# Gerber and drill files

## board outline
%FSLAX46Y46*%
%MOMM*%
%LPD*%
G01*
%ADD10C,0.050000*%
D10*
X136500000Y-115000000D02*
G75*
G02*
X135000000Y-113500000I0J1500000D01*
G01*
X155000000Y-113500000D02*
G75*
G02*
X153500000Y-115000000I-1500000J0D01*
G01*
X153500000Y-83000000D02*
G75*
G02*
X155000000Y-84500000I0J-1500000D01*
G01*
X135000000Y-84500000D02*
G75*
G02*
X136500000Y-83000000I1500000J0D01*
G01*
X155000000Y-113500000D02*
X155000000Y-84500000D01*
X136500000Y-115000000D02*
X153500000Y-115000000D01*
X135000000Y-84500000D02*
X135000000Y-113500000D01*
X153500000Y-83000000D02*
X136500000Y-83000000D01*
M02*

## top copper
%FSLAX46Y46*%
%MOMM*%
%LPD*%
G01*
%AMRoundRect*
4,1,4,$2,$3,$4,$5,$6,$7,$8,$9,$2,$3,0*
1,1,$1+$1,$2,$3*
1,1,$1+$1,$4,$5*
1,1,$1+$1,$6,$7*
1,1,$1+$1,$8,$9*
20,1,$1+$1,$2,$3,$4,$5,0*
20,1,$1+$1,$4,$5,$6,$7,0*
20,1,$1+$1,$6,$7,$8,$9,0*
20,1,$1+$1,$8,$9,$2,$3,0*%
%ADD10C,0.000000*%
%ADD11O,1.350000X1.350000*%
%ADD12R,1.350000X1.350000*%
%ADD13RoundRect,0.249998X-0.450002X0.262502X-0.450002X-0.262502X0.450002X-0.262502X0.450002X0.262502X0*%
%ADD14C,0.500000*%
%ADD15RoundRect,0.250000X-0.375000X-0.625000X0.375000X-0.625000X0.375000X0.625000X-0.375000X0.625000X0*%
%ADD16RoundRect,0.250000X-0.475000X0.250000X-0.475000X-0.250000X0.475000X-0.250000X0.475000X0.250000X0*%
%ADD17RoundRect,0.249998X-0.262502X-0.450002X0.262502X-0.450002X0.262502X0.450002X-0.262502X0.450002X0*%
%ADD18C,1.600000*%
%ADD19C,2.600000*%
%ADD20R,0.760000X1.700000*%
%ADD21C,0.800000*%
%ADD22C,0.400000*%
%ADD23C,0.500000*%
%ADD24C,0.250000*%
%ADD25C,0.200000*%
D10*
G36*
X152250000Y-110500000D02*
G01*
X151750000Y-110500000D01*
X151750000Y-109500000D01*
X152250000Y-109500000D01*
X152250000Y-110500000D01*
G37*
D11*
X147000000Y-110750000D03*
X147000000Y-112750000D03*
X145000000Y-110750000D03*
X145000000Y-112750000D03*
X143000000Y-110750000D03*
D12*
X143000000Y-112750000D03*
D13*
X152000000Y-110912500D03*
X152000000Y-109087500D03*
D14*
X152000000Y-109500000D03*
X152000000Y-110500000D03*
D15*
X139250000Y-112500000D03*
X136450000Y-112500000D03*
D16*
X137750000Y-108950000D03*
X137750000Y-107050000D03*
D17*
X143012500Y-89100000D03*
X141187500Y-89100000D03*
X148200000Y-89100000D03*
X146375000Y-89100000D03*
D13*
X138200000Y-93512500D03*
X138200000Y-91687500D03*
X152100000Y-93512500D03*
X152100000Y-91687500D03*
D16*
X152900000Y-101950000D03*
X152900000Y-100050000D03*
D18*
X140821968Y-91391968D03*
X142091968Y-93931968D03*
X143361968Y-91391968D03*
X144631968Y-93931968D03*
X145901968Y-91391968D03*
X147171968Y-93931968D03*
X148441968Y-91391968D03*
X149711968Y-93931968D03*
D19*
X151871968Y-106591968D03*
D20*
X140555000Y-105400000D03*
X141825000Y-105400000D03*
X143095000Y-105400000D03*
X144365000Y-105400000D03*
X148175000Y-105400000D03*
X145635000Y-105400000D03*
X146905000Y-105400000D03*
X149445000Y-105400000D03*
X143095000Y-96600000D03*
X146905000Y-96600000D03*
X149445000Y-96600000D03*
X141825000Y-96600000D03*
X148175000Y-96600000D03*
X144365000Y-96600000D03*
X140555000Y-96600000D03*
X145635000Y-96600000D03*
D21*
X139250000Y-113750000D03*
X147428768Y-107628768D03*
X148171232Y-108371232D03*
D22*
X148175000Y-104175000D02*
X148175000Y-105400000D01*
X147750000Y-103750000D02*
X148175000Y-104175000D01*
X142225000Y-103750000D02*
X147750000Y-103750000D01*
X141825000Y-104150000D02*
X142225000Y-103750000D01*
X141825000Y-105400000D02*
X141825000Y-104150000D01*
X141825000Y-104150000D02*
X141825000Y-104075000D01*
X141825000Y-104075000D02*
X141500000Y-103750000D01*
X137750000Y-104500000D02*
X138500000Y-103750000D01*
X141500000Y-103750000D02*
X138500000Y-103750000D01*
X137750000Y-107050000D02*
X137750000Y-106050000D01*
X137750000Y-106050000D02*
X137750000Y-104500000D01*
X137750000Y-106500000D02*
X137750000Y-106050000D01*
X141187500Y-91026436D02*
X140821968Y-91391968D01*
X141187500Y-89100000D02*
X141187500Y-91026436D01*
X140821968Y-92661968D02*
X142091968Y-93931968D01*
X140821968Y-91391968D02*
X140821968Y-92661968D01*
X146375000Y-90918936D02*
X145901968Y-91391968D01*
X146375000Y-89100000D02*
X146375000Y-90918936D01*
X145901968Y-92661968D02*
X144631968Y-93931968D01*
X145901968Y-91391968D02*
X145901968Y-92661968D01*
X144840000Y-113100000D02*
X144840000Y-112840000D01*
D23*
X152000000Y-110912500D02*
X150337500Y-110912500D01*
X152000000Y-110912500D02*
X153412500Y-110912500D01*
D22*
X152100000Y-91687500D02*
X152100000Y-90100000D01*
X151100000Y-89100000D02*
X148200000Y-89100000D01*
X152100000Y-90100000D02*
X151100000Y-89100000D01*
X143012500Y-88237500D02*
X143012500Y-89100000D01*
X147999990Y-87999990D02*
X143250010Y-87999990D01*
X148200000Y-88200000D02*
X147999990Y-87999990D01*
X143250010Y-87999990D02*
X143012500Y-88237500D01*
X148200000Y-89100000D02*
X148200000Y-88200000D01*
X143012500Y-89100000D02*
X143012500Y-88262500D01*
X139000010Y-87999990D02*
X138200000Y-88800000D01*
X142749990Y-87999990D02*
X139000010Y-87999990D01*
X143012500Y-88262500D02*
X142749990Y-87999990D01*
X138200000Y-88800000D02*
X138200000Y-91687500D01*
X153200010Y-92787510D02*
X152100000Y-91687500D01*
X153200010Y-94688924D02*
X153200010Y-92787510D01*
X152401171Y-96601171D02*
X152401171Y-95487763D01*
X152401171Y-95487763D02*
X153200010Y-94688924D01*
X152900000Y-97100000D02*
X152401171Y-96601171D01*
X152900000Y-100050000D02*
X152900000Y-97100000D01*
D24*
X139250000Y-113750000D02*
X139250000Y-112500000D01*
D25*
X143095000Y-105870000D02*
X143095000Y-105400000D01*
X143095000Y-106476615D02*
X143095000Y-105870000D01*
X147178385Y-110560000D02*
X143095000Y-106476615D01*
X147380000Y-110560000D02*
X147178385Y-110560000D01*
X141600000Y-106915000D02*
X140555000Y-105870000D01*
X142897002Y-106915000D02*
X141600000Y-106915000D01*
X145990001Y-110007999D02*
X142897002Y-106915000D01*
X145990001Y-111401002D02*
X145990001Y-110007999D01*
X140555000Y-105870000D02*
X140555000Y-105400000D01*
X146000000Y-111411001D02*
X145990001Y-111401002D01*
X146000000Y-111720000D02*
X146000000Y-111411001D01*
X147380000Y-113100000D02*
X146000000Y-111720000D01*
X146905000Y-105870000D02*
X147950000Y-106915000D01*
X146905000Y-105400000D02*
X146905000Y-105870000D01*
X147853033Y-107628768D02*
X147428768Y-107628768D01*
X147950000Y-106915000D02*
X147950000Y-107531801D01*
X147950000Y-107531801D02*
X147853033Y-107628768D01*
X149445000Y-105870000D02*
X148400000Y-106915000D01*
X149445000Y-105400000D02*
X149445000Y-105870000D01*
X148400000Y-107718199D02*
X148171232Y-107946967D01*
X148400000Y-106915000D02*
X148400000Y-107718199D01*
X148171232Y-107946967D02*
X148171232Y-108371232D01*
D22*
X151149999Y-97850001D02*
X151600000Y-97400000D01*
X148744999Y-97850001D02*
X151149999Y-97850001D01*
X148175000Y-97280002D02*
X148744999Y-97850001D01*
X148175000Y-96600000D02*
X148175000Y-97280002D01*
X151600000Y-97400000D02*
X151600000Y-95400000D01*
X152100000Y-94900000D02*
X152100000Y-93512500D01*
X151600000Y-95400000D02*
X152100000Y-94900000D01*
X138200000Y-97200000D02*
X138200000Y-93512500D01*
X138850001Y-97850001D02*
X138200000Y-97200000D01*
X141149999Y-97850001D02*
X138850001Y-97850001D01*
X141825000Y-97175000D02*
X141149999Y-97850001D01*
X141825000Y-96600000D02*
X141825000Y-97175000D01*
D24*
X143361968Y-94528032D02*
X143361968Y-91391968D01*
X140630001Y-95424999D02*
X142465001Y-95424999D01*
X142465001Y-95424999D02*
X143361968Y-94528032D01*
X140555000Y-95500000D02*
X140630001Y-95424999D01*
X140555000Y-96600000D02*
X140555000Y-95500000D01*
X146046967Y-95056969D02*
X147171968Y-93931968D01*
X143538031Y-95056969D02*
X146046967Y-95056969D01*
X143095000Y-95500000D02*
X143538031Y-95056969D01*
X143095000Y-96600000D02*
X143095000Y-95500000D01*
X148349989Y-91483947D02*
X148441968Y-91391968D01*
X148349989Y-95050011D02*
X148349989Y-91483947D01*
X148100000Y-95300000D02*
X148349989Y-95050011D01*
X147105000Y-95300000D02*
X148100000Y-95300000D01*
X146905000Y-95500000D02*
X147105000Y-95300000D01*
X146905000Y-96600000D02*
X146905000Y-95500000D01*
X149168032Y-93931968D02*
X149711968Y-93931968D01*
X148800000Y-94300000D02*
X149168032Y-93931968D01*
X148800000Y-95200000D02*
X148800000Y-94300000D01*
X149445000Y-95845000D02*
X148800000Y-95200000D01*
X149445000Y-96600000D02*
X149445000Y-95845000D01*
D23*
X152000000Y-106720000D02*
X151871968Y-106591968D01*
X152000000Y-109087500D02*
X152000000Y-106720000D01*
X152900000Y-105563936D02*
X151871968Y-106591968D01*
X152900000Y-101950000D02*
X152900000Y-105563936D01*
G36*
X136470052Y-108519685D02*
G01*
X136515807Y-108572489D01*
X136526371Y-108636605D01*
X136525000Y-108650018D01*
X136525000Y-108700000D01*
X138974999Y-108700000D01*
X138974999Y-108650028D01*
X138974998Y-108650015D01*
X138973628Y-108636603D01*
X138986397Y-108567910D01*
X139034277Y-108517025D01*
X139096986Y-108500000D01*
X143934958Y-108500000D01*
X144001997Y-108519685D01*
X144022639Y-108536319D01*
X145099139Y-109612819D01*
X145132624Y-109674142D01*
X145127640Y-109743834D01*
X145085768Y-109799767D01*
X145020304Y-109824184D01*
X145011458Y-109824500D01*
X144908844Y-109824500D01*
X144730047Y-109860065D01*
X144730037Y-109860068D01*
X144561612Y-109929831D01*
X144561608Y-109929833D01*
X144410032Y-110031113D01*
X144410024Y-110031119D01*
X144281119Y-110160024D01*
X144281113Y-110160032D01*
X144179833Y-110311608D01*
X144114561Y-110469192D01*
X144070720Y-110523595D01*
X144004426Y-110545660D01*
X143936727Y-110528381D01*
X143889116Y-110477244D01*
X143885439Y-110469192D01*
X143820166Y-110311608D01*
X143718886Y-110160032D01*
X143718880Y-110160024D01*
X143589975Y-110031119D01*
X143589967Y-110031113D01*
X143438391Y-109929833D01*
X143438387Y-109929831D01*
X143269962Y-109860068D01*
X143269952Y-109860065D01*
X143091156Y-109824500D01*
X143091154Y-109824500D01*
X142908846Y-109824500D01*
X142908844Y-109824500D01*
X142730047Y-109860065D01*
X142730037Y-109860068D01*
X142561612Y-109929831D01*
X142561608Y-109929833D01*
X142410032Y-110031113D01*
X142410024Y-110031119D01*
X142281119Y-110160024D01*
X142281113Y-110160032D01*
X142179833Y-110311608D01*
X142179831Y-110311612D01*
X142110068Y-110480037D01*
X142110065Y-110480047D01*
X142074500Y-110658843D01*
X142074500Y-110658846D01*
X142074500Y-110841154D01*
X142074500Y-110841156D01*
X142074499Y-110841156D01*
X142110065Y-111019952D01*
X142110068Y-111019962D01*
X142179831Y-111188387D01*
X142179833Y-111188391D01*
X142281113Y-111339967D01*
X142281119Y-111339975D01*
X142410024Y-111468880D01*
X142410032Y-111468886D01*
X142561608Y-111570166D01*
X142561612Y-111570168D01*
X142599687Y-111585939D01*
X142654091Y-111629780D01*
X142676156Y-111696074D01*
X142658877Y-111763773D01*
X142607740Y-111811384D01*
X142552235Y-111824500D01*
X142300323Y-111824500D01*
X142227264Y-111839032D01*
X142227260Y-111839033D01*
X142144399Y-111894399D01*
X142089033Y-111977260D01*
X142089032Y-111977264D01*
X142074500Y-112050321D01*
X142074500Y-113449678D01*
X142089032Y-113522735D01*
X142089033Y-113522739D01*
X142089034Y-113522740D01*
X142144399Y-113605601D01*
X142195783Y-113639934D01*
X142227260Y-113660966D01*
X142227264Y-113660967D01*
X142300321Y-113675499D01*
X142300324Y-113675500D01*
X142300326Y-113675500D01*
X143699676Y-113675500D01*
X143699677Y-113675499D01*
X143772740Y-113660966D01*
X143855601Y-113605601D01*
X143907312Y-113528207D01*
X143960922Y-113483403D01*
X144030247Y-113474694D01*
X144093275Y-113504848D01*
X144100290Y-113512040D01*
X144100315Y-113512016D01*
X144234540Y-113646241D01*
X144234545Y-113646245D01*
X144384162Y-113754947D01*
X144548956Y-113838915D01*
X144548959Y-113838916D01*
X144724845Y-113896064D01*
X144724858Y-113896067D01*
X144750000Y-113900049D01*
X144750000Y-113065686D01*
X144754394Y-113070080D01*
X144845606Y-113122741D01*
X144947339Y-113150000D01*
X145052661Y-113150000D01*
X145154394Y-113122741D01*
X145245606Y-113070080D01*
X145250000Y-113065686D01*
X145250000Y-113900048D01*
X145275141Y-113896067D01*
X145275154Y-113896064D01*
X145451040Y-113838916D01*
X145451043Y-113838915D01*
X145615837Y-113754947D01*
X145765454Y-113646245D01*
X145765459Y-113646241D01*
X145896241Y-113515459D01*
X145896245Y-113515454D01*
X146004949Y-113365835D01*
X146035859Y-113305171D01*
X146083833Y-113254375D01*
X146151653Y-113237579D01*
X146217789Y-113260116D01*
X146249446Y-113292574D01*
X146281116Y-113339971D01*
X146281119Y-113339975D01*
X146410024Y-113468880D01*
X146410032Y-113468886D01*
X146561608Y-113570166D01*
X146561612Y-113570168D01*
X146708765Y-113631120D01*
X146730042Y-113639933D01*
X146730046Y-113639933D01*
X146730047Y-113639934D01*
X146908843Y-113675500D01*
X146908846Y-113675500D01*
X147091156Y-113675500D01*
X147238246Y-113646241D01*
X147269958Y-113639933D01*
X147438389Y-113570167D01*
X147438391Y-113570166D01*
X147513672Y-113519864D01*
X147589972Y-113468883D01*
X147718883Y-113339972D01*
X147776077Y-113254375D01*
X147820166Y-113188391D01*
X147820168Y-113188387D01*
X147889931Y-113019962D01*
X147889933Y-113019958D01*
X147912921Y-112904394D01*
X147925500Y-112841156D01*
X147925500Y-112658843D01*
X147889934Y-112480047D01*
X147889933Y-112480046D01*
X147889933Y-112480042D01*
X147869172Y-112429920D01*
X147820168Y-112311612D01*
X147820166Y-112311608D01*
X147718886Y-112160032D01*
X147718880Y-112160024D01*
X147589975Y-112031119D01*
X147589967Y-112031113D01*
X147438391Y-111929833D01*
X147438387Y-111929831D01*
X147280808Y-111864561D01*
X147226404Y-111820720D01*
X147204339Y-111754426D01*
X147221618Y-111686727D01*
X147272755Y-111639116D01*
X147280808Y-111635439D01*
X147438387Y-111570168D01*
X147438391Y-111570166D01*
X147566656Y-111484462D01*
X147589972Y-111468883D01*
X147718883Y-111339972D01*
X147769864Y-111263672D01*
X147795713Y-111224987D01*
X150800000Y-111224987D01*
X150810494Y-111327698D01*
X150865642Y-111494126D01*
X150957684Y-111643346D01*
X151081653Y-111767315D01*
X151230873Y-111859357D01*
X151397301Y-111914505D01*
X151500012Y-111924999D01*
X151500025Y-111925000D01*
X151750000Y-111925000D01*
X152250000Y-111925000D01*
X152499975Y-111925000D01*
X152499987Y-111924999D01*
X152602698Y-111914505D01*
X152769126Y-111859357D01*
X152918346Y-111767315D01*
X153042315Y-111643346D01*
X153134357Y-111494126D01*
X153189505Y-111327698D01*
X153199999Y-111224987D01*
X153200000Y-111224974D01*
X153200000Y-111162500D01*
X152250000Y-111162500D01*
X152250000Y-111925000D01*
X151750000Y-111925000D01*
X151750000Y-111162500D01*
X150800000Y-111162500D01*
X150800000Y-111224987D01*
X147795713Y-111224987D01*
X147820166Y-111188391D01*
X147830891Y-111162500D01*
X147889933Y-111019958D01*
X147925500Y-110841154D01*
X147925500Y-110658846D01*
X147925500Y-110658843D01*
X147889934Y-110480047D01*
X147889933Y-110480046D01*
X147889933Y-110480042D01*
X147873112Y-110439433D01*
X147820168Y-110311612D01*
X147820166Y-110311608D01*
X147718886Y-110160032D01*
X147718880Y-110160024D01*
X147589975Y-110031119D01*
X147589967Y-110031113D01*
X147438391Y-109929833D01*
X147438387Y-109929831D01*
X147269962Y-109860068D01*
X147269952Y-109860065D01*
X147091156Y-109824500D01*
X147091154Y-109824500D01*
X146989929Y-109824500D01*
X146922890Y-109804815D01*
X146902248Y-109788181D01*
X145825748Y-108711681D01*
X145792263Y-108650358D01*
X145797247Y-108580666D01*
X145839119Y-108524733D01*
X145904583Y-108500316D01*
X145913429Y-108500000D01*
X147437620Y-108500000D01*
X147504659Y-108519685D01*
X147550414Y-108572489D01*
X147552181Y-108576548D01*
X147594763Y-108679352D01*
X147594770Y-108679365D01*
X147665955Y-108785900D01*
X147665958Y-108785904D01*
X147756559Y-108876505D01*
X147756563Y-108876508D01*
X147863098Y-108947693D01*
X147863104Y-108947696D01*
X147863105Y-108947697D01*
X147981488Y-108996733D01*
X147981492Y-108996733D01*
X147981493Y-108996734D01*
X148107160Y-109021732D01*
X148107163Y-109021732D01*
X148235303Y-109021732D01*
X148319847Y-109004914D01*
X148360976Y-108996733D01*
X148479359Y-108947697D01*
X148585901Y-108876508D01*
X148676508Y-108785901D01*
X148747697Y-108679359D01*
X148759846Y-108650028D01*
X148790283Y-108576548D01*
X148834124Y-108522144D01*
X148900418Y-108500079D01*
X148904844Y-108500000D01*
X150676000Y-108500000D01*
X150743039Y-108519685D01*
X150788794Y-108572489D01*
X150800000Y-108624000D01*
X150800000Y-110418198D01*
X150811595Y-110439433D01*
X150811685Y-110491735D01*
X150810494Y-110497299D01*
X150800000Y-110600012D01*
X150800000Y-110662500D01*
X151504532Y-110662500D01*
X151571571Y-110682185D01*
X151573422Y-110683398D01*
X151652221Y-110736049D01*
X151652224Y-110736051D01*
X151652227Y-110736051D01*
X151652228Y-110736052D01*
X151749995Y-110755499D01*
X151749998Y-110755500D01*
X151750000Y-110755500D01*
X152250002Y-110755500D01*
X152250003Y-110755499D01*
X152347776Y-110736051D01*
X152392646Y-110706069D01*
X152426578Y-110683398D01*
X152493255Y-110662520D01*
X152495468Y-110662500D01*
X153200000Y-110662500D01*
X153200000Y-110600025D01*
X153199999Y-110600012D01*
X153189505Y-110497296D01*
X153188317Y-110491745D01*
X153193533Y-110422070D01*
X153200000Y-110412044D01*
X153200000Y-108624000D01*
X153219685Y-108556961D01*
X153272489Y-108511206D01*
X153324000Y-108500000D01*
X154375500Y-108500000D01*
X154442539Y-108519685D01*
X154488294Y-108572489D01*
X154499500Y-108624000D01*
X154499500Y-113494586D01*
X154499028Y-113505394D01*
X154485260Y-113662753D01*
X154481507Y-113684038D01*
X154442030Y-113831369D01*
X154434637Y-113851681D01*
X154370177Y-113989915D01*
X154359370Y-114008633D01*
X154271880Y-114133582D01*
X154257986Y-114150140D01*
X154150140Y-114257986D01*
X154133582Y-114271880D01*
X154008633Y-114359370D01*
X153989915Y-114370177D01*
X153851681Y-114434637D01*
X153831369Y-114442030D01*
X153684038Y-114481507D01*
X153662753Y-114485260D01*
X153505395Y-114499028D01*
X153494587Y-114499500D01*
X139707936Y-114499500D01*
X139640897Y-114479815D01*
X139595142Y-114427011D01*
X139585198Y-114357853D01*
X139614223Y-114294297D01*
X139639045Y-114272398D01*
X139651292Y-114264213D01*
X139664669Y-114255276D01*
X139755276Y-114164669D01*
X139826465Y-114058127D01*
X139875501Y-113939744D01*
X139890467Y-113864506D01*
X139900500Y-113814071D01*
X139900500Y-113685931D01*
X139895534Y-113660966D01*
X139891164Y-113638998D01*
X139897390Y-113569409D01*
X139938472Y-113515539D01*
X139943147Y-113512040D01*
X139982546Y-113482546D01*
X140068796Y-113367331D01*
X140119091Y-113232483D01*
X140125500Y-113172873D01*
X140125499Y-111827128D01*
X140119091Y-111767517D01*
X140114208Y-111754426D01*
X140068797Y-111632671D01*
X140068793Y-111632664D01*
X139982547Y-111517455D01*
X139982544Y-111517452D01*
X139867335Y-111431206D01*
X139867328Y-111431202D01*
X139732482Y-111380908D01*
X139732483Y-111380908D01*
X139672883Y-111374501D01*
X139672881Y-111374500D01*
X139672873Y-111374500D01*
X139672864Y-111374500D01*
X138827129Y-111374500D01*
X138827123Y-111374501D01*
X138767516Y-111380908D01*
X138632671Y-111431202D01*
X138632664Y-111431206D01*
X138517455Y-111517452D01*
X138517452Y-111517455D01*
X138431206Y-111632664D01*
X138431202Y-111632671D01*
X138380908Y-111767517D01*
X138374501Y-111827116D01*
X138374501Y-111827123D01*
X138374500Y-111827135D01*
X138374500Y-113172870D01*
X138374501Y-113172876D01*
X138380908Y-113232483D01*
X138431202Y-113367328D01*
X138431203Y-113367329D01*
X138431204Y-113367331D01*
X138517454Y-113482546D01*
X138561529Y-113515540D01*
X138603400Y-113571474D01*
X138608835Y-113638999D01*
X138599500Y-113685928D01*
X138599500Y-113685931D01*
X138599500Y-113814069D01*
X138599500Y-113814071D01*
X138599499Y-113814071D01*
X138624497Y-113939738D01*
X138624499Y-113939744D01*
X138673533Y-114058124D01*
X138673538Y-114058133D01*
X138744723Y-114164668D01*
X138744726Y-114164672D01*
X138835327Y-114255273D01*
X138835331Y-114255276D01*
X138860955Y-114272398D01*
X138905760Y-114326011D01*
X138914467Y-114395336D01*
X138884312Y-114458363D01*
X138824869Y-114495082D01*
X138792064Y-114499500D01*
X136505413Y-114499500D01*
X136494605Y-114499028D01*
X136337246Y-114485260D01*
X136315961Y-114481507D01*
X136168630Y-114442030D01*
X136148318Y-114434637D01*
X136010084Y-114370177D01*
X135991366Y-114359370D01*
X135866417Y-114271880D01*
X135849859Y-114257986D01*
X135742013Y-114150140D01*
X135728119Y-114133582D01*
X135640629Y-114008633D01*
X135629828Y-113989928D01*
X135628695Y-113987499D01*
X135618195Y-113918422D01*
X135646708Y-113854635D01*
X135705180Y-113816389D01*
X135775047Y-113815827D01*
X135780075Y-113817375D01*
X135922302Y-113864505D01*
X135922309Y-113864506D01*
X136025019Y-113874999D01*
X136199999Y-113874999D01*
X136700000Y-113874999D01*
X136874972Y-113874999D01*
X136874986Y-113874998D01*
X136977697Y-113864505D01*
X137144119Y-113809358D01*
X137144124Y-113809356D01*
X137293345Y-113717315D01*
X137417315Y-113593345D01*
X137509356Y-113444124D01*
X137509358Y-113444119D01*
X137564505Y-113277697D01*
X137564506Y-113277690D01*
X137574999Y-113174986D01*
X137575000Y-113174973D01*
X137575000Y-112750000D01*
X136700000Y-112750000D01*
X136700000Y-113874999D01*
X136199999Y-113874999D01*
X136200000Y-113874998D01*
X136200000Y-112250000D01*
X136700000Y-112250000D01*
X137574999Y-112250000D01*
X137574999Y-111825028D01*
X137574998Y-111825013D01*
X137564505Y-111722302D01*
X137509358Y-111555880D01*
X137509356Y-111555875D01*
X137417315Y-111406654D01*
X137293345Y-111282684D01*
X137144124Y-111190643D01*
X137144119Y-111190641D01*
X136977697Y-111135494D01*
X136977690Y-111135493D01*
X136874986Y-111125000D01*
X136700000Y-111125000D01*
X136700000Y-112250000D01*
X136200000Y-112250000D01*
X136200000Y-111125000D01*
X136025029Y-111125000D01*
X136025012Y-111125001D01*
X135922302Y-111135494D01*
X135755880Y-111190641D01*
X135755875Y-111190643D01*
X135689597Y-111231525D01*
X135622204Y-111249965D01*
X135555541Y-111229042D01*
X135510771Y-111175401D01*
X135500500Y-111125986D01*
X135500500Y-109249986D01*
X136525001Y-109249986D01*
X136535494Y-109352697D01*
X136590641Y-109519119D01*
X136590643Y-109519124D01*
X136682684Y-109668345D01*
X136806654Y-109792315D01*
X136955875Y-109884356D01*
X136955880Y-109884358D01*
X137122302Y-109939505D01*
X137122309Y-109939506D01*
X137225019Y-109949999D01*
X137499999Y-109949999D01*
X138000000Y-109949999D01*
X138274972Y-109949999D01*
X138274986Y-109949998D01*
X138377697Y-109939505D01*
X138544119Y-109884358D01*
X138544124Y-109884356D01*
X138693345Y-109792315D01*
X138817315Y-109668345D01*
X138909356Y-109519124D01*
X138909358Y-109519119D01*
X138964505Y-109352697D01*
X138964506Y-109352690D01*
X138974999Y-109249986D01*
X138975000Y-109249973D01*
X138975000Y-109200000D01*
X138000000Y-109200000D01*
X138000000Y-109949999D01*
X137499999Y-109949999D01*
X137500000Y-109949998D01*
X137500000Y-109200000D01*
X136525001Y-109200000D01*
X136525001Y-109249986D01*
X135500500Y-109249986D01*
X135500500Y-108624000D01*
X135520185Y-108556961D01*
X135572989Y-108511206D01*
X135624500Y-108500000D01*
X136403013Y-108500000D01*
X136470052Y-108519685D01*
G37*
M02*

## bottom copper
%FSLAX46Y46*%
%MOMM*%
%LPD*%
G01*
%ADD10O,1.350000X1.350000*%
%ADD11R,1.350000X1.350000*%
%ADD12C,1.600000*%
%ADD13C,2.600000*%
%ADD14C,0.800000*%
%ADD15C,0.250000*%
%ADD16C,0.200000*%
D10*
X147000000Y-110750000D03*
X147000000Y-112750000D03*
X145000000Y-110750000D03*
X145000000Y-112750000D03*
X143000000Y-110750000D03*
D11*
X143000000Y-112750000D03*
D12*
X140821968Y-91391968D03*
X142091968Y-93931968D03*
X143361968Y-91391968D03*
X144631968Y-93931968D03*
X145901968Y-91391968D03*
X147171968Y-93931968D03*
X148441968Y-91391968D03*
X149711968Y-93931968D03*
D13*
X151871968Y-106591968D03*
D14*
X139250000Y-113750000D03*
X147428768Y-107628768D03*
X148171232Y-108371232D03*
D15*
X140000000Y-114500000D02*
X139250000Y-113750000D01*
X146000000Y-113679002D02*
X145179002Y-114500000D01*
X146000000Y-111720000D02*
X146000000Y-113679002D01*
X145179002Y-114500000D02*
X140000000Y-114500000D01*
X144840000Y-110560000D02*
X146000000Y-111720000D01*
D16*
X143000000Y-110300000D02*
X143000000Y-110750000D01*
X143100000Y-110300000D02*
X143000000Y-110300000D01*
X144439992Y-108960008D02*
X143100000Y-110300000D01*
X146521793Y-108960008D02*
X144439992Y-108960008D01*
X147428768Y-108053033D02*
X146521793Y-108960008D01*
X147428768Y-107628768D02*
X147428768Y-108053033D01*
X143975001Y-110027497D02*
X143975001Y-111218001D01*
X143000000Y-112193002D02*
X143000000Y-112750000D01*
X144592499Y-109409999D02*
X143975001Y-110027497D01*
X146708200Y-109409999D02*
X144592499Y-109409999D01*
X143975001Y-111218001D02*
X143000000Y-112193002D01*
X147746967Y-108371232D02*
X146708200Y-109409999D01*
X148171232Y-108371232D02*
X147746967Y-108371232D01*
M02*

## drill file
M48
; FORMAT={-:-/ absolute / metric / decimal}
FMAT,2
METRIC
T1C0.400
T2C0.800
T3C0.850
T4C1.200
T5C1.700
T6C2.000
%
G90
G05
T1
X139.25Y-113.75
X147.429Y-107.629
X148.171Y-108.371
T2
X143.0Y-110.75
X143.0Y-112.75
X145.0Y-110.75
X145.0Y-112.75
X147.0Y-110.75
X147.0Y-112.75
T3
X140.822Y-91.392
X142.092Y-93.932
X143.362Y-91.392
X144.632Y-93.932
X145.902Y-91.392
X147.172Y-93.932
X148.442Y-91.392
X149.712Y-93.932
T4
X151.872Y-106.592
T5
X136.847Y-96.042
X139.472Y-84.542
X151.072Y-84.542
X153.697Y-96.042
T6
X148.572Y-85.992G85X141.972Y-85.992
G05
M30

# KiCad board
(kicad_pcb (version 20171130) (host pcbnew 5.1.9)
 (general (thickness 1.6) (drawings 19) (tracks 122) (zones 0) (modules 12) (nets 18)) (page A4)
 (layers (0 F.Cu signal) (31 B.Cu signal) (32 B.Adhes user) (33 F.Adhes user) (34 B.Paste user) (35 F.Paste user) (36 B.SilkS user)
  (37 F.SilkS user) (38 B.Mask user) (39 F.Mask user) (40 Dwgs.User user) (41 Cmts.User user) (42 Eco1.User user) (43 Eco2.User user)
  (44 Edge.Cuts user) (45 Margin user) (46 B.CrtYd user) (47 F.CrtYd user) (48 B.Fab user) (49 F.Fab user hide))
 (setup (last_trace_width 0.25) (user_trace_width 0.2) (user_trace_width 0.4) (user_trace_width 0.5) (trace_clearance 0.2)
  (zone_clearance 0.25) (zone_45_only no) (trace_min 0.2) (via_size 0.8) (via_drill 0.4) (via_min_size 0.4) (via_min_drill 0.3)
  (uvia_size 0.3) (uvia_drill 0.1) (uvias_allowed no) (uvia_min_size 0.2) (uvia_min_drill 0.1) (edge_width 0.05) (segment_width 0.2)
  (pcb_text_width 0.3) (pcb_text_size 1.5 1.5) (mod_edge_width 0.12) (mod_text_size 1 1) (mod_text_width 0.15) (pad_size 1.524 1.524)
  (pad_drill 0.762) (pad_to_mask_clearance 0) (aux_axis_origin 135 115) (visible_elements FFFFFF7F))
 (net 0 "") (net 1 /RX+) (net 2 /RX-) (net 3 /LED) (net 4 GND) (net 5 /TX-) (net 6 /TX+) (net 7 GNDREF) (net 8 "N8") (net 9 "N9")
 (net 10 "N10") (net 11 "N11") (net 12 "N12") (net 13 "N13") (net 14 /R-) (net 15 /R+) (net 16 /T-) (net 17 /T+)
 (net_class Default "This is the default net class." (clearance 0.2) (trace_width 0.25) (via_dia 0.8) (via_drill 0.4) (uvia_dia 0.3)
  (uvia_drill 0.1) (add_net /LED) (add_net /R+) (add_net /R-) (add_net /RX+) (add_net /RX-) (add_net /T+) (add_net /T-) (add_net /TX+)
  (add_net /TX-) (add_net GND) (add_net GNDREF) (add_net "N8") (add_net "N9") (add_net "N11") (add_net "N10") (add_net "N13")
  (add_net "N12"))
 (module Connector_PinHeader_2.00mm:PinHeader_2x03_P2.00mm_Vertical (layer F.Cu) (at 143 112.75 90)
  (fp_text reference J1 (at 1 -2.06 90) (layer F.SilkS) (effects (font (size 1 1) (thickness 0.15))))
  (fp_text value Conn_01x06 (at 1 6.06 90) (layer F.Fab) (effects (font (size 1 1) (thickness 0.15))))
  (pad 6 thru_hole oval (at 2 4 90) (size 1.35 1.35) (drill 0.8) (layers *.Cu *.Mask) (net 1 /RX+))
  (pad 5 thru_hole oval (at 0 4 90) (size 1.35 1.35) (drill 0.8) (layers *.Cu *.Mask) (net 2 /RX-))
  (pad 4 thru_hole oval (at 2 2 90) (size 1.35 1.35) (drill 0.8) (layers *.Cu *.Mask) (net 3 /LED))
  (pad 3 thru_hole oval (at 0 2 90) (size 1.35 1.35) (drill 0.8) (layers *.Cu *.Mask) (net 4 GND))
  (pad 2 thru_hole oval (at 2 0 90) (size 1.35 1.35) (drill 0.8) (layers *.Cu *.Mask) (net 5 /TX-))
  (pad 1 thru_hole rect (at 0 0 90) (size 1.35 1.35) (drill 0.8) (layers *.Cu *.Mask) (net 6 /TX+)))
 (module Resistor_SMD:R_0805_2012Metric (layer F.Cu) (at 152 110 270)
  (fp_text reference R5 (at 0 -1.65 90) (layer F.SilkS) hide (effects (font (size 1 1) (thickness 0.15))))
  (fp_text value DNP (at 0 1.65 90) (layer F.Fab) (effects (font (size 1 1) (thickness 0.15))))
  (pad 2 smd roundrect (at 0.9125 0 270) (size 1.025 1.4) (layers F.Cu F.Paste F.Mask) (roundrect_rratio 0.2439004878048781) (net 4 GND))
  (pad 1 smd roundrect (at -0.9125 0 270) (size 1.025 1.4) (layers F.Cu F.Paste F.Mask) (roundrect_rratio 0.2439004878048781) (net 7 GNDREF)))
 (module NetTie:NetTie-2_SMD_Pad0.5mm (layer F.Cu) (at 152 110 90)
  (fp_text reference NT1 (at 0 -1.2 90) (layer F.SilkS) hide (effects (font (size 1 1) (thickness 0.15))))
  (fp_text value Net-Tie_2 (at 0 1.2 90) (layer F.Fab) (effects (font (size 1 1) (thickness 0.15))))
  (fp_poly (pts (xy -0.5 -0.25) (xy 0.5 -0.25) (xy 0.5 0.25) (xy -0.5 0.25)) (layer F.Cu) (width 0))
  (pad 2 smd circle (at 0.5 0 90) (size 0.5 0.5) (layers F.Cu) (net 7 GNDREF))
  (pad 1 smd circle (at -0.5 0 90) (size 0.5 0.5) (layers F.Cu) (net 4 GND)))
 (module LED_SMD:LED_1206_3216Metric (layer F.Cu) (at 137.85 112.5)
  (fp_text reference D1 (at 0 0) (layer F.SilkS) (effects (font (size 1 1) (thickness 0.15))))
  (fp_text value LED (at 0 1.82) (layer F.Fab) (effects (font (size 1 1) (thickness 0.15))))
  (pad 2 smd roundrect (at 1.4 0) (size 1.25 1.75) (layers F.Cu F.Paste F.Mask) (roundrect_rratio 0.2) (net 3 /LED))
  (pad 1 smd roundrect (at -1.4 0) (size 1.25 1.75) (layers F.Cu F.Paste F.Mask) (roundrect_rratio 0.2) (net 4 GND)))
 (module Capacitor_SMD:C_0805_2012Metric (layer F.Cu) (at 137.75 108 270)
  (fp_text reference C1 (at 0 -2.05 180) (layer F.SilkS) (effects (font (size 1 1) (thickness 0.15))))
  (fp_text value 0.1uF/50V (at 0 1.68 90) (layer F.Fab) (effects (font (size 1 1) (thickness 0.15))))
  (pad 2 smd roundrect (at 0.95 0 270) (size 1 1.45) (layers F.Cu F.Paste F.Mask) (roundrect_rratio 0.25) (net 4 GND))
  (pad 1 smd roundrect (at -0.95 0 270) (size 1 1.45) (layers F.Cu F.Paste F.Mask) (roundrect_rratio 0.25) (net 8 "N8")))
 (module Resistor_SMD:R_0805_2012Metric (layer F.Cu) (at 142.1 89.1)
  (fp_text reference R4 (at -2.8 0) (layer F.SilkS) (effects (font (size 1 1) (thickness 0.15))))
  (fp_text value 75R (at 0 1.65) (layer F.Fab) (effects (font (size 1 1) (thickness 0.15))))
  (pad 2 smd roundrect (at 0.9125 0) (size 1.025 1.4) (layers F.Cu F.Paste F.Mask) (roundrect_rratio 0.2439004878048781) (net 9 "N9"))
  (pad 1 smd roundrect (at -0.9125 0) (size 1.025 1.4) (layers F.Cu F.Paste F.Mask) (roundrect_rratio 0.2439004878048781) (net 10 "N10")))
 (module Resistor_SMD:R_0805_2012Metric (layer F.Cu) (at 147.2875 89.1)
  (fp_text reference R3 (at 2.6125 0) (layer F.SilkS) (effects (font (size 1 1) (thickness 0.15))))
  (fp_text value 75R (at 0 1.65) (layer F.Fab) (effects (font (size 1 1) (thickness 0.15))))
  (pad 2 smd roundrect (at 0.9125 0) (size 1.025 1.4) (layers F.Cu F.Paste F.Mask) (roundrect_rratio 0.2439004878048781) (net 9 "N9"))
  (pad 1 smd roundrect (at -0.9125 0) (size 1.025 1.4) (layers F.Cu F.Paste F.Mask) (roundrect_rratio 0.2439004878048781) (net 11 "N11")))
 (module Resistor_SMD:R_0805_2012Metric (layer F.Cu) (at 138.2 92.6 270)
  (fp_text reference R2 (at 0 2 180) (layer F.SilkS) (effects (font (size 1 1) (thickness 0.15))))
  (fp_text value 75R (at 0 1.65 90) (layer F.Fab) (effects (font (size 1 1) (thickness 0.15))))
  (pad 2 smd roundrect (at 0.9125 0 270) (size 1.025 1.4) (layers F.Cu F.Paste F.Mask) (roundrect_rratio 0.2439004878048781) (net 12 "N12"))
  (pad 1 smd roundrect (at -0.9125 0 270) (size 1.025 1.4) (layers F.Cu F.Paste F.Mask) (roundrect_rratio 0.2439004878048781) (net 9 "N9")))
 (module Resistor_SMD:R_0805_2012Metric (layer F.Cu) (at 152.1 92.6 270)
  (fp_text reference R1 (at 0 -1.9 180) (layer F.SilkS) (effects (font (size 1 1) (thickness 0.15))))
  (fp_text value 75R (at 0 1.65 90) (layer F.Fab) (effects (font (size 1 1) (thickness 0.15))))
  (pad 2 smd roundrect (at 0.9125 0 270) (size 1.025 1.4) (layers F.Cu F.Paste F.Mask) (roundrect_rratio 0.2439004878048781) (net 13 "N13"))
  (pad 1 smd roundrect (at -0.9125 0 270) (size 1.025 1.4) (layers F.Cu F.Paste F.Mask) (roundrect_rratio 0.2439004878048781) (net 9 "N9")))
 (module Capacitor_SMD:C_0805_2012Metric (layer F.Cu) (at 152.9 101 270)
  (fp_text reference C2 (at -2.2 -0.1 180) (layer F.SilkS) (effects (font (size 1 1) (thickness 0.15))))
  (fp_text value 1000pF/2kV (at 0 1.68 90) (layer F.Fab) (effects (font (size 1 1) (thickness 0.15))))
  (pad 2 smd roundrect (at 0.95 0 270) (size 1 1.45) (layers F.Cu F.Paste F.Mask) (roundrect_rratio 0.25) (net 7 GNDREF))
  (pad 1 smd roundrect (at -0.95 0 270) (size 1 1.45) (layers F.Cu F.Paste F.Mask) (roundrect_rratio 0.25) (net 9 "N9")))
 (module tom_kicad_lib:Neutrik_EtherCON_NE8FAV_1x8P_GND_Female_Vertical (layer B.Cu) (at 145.271968 96.041968 180)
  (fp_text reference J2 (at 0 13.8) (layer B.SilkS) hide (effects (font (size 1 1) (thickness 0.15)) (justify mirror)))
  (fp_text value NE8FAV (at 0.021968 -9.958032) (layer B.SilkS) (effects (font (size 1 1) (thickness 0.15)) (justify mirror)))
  (pad "" np_thru_hole oval (at 0 10.05 180) (size 8.6 2) (drill oval 8.6 2) (layers *.Cu *.Mask))
  (pad "" np_thru_hole circle (at 5.8 11.5 180) (size 1.7 1.7) (drill 1.7) (layers *.Cu *.Mask))
  (pad "" np_thru_hole circle (at -5.8 11.5 180) (size 1.7 1.7) (drill 1.7) (layers *.Cu *.Mask))
  (pad "" np_thru_hole circle (at -8.425 0 180) (size 1.7 1.7) (drill 1.7) (layers *.Cu *.Mask))
  (pad "" np_thru_hole circle (at 8.425 0 180) (size 1.7 1.7) (drill 1.7) (layers *.Cu *.Mask))
  (pad 8 thru_hole circle (at 4.45 4.65 180) (size 1.6 1.6) (drill 0.85) (layers *.Cu *.Mask) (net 10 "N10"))
  (pad 7 thru_hole circle (at 3.18 2.11 180) (size 1.6 1.6) (drill 0.85) (layers *.Cu *.Mask) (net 10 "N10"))
  (pad 6 thru_hole circle (at 1.91 4.65 180) (size 1.6 1.6) (drill 0.85) (layers *.Cu *.Mask) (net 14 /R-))
  (pad 5 thru_hole circle (at 0.64 2.11 180) (size 1.6 1.6) (drill 0.85) (layers *.Cu *.Mask) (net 11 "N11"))
  (pad 4 thru_hole circle (at -0.63 4.65 180) (size 1.6 1.6) (drill 0.85) (layers *.Cu *.Mask) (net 11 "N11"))
  (pad 3 thru_hole circle (at -1.9 2.11 180) (size 1.6 1.6) (drill 0.85) (layers *.Cu *.Mask) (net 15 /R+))
  (pad 2 thru_hole circle (at -3.17 4.65 180) (size 1.6 1.6) (drill 0.85) (layers *.Cu *.Mask) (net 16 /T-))
  (pad 1 thru_hole circle (at -4.44 2.11 180) (size 1.6 1.6) (drill 0.85) (layers *.Cu *.Mask) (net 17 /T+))
  (pad SH thru_hole circle (at -6.6 -10.55 180) (size 2.6 2.6) (drill 1.2) (layers *.Cu *.Mask) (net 7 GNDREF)))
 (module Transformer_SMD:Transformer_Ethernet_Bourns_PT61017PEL (layer F.Cu) (at 145 101 90)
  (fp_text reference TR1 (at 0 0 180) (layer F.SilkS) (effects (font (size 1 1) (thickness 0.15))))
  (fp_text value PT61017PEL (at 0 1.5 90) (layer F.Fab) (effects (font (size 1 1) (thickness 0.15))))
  (pad 1 smd rect (at -4.4 -4.445 90) (size 1.7 0.76) (layers F.Cu F.Paste F.Mask) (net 2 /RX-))
  (pad 2 smd rect (at -4.4 -3.175 90) (size 1.7 0.76) (layers F.Cu F.Paste F.Mask) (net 8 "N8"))
  (pad 3 smd rect (at -4.4 -1.905 90) (size 1.7 0.76) (layers F.Cu F.Paste F.Mask) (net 1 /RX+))
  (pad 4 smd rect (at -4.4 -0.635 90) (size 1.7 0.76) (layers F.Cu F.Paste F.Mask))
  (pad 7 smd rect (at -4.4 3.175 90) (size 1.7 0.76) (layers F.Cu F.Paste F.Mask) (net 8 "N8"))
  (pad 5 smd rect (at -4.4 0.635 90) (size 1.7 0.76) (layers F.Cu F.Paste F.Mask))
  (pad 6 smd rect (at -4.4 1.905 90) (size 1.7 0.76) (layers F.Cu F.Paste F.Mask) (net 5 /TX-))
  (pad 8 smd rect (at -4.4 4.445 90) (size 1.7 0.76) (layers F.Cu F.Paste F.Mask) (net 6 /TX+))
  (pad 14 smd rect (at 4.4 -1.905 90) (size 1.7 0.76) (layers F.Cu F.Paste F.Mask) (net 15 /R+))
  (pad 11 smd rect (at 4.4 1.905 90) (size 1.7 0.76) (layers F.Cu F.Paste F.Mask) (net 16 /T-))
  (pad 9 smd rect (at 4.4 4.445 90) (size 1.7 0.76) (layers F.Cu F.Paste F.Mask) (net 17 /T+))
  (pad 15 smd rect (at 4.4 -3.175 90) (size 1.7 0.76) (layers F.Cu F.Paste F.Mask) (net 12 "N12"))
  (pad 10 smd rect (at 4.4 3.175 90) (size 1.7 0.76) (layers F.Cu F.Paste F.Mask) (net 13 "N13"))
  (pad 13 smd rect (at 4.4 -0.635 90) (size 1.7 0.76) (layers F.Cu F.Paste F.Mask))
  (pad 16 smd rect (at 4.4 -4.445 90) (size 1.7 0.76) (layers F.Cu F.Paste F.Mask) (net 14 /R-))
  (pad 12 smd rect (at 4.4 0.635 90) (size 1.7 0.76) (layers F.Cu F.Paste F.Mask)))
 (gr_arc (start 136.5 113.5) (end 135 113.5) (angle -90) (layer Edge.Cuts) (width 0.05))
 (gr_arc (start 153.5 113.5) (end 153.5 115) (angle -90) (layer Edge.Cuts) (width 0.05))
 (gr_arc (start 153.5 84.5) (end 155 84.5) (angle -90) (layer Edge.Cuts) (width 0.05))
 (gr_arc (start 136.5 84.5) (end 136.5 83) (angle -90) (layer Edge.Cuts) (width 0.05))
 (gr_line (start 155 113.5) (end 155 84.5) (layer Edge.Cuts) (width 0.05))
 (gr_line (start 136.5 115) (end 153.5 115) (layer Edge.Cuts) (width 0.05))
 (gr_line (start 135 84.5) (end 135 113.5) (layer Edge.Cuts) (width 0.05))
 (gr_line (start 153.5 83) (end 136.5 83) (layer Edge.Cuts) (width 0.05))
 (segment (start 148.175 104.175) (end 148.175 105.4) (width 0.4) (layer F.Cu) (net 8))
 (segment (start 147.75 103.75) (end 148.175 104.175) (width 0.4) (layer F.Cu) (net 8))
 (segment (start 142.225 103.75) (end 147.75 103.75) (width 0.4) (layer F.Cu) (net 8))
 (segment (start 141.825 104.15) (end 142.225 103.75) (width 0.4) (layer F.Cu) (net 8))
 (segment (start 141.825 105.4) (end 141.825 104.15) (width 0.4) (layer F.Cu) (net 8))
 (segment (start 141.825 104.15) (end 141.825 104.075) (width 0.4) (layer F.Cu) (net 8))
 (segment (start 141.825 104.075) (end 141.5 103.75) (width 0.4) (layer F.Cu) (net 8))
 (segment (start 137.75 104.5) (end 138.5 103.75) (width 0.4) (layer F.Cu) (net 8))
 (segment (start 141.5 103.75) (end 138.5 103.75) (width 0.4) (layer F.Cu) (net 8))
 (segment (start 137.75 107.05) (end 137.75 106.05) (width 0.4) (layer F.Cu) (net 8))
 (segment (start 137.75 106.05) (end 137.75 104.5) (width 0.4) (layer F.Cu) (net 8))
 (segment (start 137.75 106.5) (end 137.75 106.05) (width 0.4) (layer F.Cu) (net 8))
 (segment (start 141.1875 91.026436) (end 140.821968 91.391968) (width 0.4) (layer F.Cu) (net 10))
 (segment (start 141.1875 89.1) (end 141.1875 91.026436) (width 0.4) (layer F.Cu) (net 10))
 (segment (start 140.821968 92.661968) (end 142.091968 93.931968) (width 0.4) (layer F.Cu) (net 10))
 (segment (start 140.821968 91.391968) (end 140.821968 92.661968) (width 0.4) (layer F.Cu) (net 10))
 (segment (start 146.375 90.918936) (end 145.901968 91.391968) (width 0.4) (layer F.Cu) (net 11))
 (segment (start 146.375 89.1) (end 146.375 90.918936) (width 0.4) (layer F.Cu) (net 11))
 (segment (start 145.901968 92.661968) (end 144.631968 93.931968) (width 0.4) (layer F.Cu) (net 11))
 (segment (start 145.901968 91.391968) (end 145.901968 92.661968) (width 0.4) (layer F.Cu) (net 11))
 (segment (start 144.84 113.1) (end 144.84 112.84) (width 0.4) (layer F.Cu) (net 4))
 (segment (start 152 110.9125) (end 150.3375 110.9125) (width 0.5) (layer F.Cu) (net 4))
 (segment (start 152 110.9125) (end 153.4125 110.9125) (width 0.5) (layer F.Cu) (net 4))
 (segment (start 152.1 91.6875) (end 152.1 90.1) (width 0.4) (layer F.Cu) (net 9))
 (segment (start 151.1 89.1) (end 148.2 89.1) (width 0.4) (layer F.Cu) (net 9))
 (segment (start 152.1 90.1) (end 151.1 89.1) (width 0.4) (layer F.Cu) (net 9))
 (segment (start 143.0125 88.2375) (end 143.0125 89.1) (width 0.4) (layer F.Cu) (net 9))
 (segment (start 147.99999 87.99999) (end 143.25001 87.99999) (width 0.4) (layer F.Cu) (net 9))
 (segment (start 148.2 88.2) (end 147.99999 87.99999) (width 0.4) (layer F.Cu) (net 9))
 (segment (start 143.25001 87.99999) (end 143.0125 88.2375) (width 0.4) (layer F.Cu) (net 9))
 (segment (start 148.2 89.1) (end 148.2 88.2) (width 0.4) (layer F.Cu) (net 9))
 (segment (start 143.0125 89.1) (end 143.0125 88.2625) (width 0.4) (layer F.Cu) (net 9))
 (segment (start 139.00001 87.99999) (end 138.2 88.8) (width 0.4) (layer F.Cu) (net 9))
 (segment (start 142.74999 87.99999) (end 139.00001 87.99999) (width 0.4) (layer F.Cu) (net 9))
 (segment (start 143.0125 88.2625) (end 142.74999 87.99999) (width 0.4) (layer F.Cu) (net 9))
 (segment (start 138.2 88.8) (end 138.2 91.6875) (width 0.4) (layer F.Cu) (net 9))
 (segment (start 153.20001 92.78751) (end 152.1 91.6875) (width 0.4) (layer F.Cu) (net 9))
 (segment (start 153.20001 94.688924) (end 153.20001 92.78751) (width 0.4) (layer F.Cu) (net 9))
 (segment (start 152.401171 96.601171) (end 152.401171 95.487763) (width 0.4) (layer F.Cu) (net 9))
 (segment (start 152.401171 95.487763) (end 153.20001 94.688924) (width 0.4) (layer F.Cu) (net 9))
 (segment (start 152.9 97.1) (end 152.401171 96.601171) (width 0.4) (layer F.Cu) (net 9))
 (segment (start 152.9 100.05) (end 152.9 97.1) (width 0.4) (layer F.Cu) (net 9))
 (via (at 139.25 113.75) (size 0.8) (drill 0.4) (layers F.Cu B.Cu) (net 3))
 (segment (start 139.25 113.75) (end 139.25 112.5) (width 0.25) (layer F.Cu) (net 3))
 (segment (start 140 114.5) (end 139.25 113.75) (width 0.25) (layer B.Cu) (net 3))
 (segment (start 146 113.679002) (end 145.179002 114.5) (width 0.25) (layer B.Cu) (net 3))
 (segment (start 146 111.72) (end 146 113.679002) (width 0.25) (layer B.Cu) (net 3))
 (segment (start 145.179002 114.5) (end 140 114.5) (width 0.25) (layer B.Cu) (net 3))
 (segment (start 144.84 110.56) (end 146 111.72) (width 0.25) (layer B.Cu) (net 3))
 (segment (start 143.095 105.87) (end 143.095 105.4) (width 0.2) (layer F.Cu) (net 1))
 (segment (start 143.095 106.476615) (end 143.095 105.87) (width 0.2) (layer F.Cu) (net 1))
 (segment (start 147.178385 110.56) (end 143.095 106.476615) (width 0.2) (layer F.Cu) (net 1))
 (segment (start 147.38 110.56) (end 147.178385 110.56) (width 0.2) (layer F.Cu) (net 1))
 (segment (start 141.6 106.915) (end 140.555 105.87) (width 0.2) (layer F.Cu) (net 2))
 (segment (start 142.897002 106.915) (end 141.6 106.915) (width 0.2) (layer F.Cu) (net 2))
 (segment (start 145.990001 110.007999) (end 142.897002 106.915) (width 0.2) (layer F.Cu) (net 2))
 (segment (start 145.990001 111.401002) (end 145.990001 110.007999) (width 0.2) (layer F.Cu) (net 2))
 (segment (start 140.555 105.87) (end 140.555 105.4) (width 0.2) (layer F.Cu) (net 2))
 (segment (start 146 111.411001) (end 145.990001 111.401002) (width 0.2) (layer F.Cu) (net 2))
 (segment (start 146 111.72) (end 146 111.411001) (width 0.2) (layer F.Cu) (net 2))
 (segment (start 147.38 113.1) (end 146 111.72) (width 0.2) (layer F.Cu) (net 2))
 (segment (start 146.905 105.87) (end 147.95 106.915) (width 0.2) (layer F.Cu) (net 5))
 (segment (start 146.905 105.4) (end 146.905 105.87) (width 0.2) (layer F.Cu) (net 5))
 (segment (start 147.853033 107.628768) (end 147.428768 107.628768) (width 0.2) (layer F.Cu) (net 5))
 (segment (start 147.95 106.915) (end 147.95 107.531801) (width 0.2) (layer F.Cu) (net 5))
 (segment (start 147.95 107.531801) (end 147.853033 107.628768) (width 0.2) (layer F.Cu) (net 5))
 (via (at 147.428768 107.628768) (size 0.8) (drill 0.4) (layers F.Cu B.Cu) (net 5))
 (segment (start 143 110.3) (end 143 110.75) (width 0.2) (layer B.Cu) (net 5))
 (segment (start 143.1 110.3) (end 143 110.3) (width 0.2) (layer B.Cu) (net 5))
 (segment (start 144.439992 108.960008) (end 143.1 110.3) (width 0.2) (layer B.Cu) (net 5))
 (segment (start 146.521793 108.960008) (end 144.439992 108.960008) (width 0.2) (layer B.Cu) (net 5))
 (segment (start 147.428768 108.053033) (end 146.521793 108.960008) (width 0.2) (layer B.Cu) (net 5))
 (segment (start 147.428768 107.628768) (end 147.428768 108.053033) (width 0.2) (layer B.Cu) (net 5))
 (segment (start 149.445 105.87) (end 148.4 106.915) (width 0.2) (layer F.Cu) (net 6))
 (segment (start 149.445 105.4) (end 149.445 105.87) (width 0.2) (layer F.Cu) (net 6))
 (segment (start 148.4 107.718199) (end 148.171232 107.946967) (width 0.2) (layer F.Cu) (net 6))
 (segment (start 148.4 106.915) (end 148.4 107.718199) (width 0.2) (layer F.Cu) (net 6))
 (segment (start 148.171232 107.946967) (end 148.171232 108.371232) (width 0.2) (layer F.Cu) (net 6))
 (via (at 148.171232 108.371232) (size 0.8) (drill 0.4) (layers F.Cu B.Cu) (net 6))
 (segment (start 143.975001 110.027497) (end 143.975001 111.218001) (width 0.2) (layer B.Cu) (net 6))
 (segment (start 143 112.193002) (end 143 112.75) (width 0.2) (layer B.Cu) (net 6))
 (segment (start 144.592499 109.409999) (end 143.975001 110.027497) (width 0.2) (layer B.Cu) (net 6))
 (segment (start 146.7082 109.409999) (end 144.592499 109.409999) (width 0.2) (layer B.Cu) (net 6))
 (segment (start 143.975001 111.218001) (end 143 112.193002) (width 0.2) (layer B.Cu) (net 6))
 (segment (start 147.746967 108.371232) (end 146.7082 109.409999) (width 0.2) (layer B.Cu) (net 6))
 (segment (start 148.171232 108.371232) (end 147.746967 108.371232) (width 0.2) (layer B.Cu) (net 6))
 (segment (start 151.149999 97.850001) (end 151.6 97.4) (width 0.4) (layer F.Cu) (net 13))
 (segment (start 148.744999 97.850001) (end 151.149999 97.850001) (width 0.4) (layer F.Cu) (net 13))
 (segment (start 148.175 97.280002) (end 148.744999 97.850001) (width 0.4) (layer F.Cu) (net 13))
 (segment (start 148.175 96.6) (end 148.175 97.280002) (width 0.4) (layer F.Cu) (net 13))
 (segment (start 151.6 97.4) (end 151.6 95.4) (width 0.4) (layer F.Cu) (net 13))
 (segment (start 152.1 94.9) (end 152.1 93.5125) (width 0.4) (layer F.Cu) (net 13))
 (segment (start 151.6 95.4) (end 152.1 94.9) (width 0.4) (layer F.Cu) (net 13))
 (segment (start 138.2 97.2) (end 138.2 93.5125) (width 0.4) (layer F.Cu) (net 12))
 (segment (start 138.850001 97.850001) (end 138.2 97.2) (width 0.4) (layer F.Cu) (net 12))
 (segment (start 141.149999 97.850001) (end 138.850001 97.850001) (width 0.4) (layer F.Cu) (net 12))
 (segment (start 141.825 97.175) (end 141.149999 97.850001) (width 0.4) (layer F.Cu) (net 12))
 (segment (start 141.825 96.6) (end 141.825 97.175) (width 0.4) (layer F.Cu) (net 12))
 (segment (start 143.361968 94.528032) (end 143.361968 91.391968) (width 0.25) (layer F.Cu) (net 14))
 (segment (start 140.630001 95.424999) (end 142.465001 95.424999) (width 0.25) (layer F.Cu) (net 14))
 (segment (start 142.465001 95.424999) (end 143.361968 94.528032) (width 0.25) (layer F.Cu) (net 14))
 (segment (start 140.555 95.5) (end 140.630001 95.424999) (width 0.25) (layer F.Cu) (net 14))
 (segment (start 140.555 96.6) (end 140.555 95.5) (width 0.25) (layer F.Cu) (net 14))
 (segment (start 146.046967 95.056969) (end 147.171968 93.931968) (width 0.25) (layer F.Cu) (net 15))
 (segment (start 143.538031 95.056969) (end 146.046967 95.056969) (width 0.25) (layer F.Cu) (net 15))
 (segment (start 143.095 95.5) (end 143.538031 95.056969) (width 0.25) (layer F.Cu) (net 15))
 (segment (start 143.095 96.6) (end 143.095 95.5) (width 0.25) (layer F.Cu) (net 15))
 (segment (start 148.349989 91.483947) (end 148.441968 91.391968) (width 0.25) (layer F.Cu) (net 16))
 (segment (start 148.349989 95.050011) (end 148.349989 91.483947) (width 0.25) (layer F.Cu) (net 16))
 (segment (start 148.1 95.3) (end 148.349989 95.050011) (width 0.25) (layer F.Cu) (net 16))
 (segment (start 147.105 95.3) (end 148.1 95.3) (width 0.25) (layer F.Cu) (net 16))
 (segment (start 146.905 95.5) (end 147.105 95.3) (width 0.25) (layer F.Cu) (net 16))
 (segment (start 146.905 96.6) (end 146.905 95.5) (width 0.25) (layer F.Cu) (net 16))
 (segment (start 149.168032 93.931968) (end 149.711968 93.931968) (width 0.25) (layer F.Cu) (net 17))
 (segment (start 148.8 94.3) (end 149.168032 93.931968) (width 0.25) (layer F.Cu) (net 17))
 (segment (start 148.8 95.2) (end 148.8 94.3) (width 0.25) (layer F.Cu) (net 17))
 (segment (start 149.445 95.845) (end 148.8 95.2) (width 0.25) (layer F.Cu) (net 17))
 (segment (start 149.445 96.6) (end 149.445 95.845) (width 0.25) (layer F.Cu) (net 17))
 (segment (start 152 106.72) (end 151.871968 106.591968) (width 0.5) (layer F.Cu) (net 7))
 (segment (start 152 109.0875) (end 152 106.72) (width 0.5) (layer F.Cu) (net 7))
 (segment (start 152.9 105.563936) (end 151.871968 106.591968) (width 0.5) (layer F.Cu) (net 7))
 (segment (start 152.9 101.95) (end 152.9 105.563936) (width 0.5) (layer F.Cu) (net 7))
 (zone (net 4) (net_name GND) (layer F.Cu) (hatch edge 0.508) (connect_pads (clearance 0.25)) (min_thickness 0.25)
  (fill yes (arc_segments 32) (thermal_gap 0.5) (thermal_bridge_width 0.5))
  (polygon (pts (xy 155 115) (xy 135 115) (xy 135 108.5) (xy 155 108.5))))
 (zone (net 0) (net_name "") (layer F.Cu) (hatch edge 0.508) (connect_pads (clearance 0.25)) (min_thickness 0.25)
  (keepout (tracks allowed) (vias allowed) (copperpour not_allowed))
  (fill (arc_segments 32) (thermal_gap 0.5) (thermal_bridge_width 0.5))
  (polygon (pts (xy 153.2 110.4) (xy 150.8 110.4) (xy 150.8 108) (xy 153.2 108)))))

